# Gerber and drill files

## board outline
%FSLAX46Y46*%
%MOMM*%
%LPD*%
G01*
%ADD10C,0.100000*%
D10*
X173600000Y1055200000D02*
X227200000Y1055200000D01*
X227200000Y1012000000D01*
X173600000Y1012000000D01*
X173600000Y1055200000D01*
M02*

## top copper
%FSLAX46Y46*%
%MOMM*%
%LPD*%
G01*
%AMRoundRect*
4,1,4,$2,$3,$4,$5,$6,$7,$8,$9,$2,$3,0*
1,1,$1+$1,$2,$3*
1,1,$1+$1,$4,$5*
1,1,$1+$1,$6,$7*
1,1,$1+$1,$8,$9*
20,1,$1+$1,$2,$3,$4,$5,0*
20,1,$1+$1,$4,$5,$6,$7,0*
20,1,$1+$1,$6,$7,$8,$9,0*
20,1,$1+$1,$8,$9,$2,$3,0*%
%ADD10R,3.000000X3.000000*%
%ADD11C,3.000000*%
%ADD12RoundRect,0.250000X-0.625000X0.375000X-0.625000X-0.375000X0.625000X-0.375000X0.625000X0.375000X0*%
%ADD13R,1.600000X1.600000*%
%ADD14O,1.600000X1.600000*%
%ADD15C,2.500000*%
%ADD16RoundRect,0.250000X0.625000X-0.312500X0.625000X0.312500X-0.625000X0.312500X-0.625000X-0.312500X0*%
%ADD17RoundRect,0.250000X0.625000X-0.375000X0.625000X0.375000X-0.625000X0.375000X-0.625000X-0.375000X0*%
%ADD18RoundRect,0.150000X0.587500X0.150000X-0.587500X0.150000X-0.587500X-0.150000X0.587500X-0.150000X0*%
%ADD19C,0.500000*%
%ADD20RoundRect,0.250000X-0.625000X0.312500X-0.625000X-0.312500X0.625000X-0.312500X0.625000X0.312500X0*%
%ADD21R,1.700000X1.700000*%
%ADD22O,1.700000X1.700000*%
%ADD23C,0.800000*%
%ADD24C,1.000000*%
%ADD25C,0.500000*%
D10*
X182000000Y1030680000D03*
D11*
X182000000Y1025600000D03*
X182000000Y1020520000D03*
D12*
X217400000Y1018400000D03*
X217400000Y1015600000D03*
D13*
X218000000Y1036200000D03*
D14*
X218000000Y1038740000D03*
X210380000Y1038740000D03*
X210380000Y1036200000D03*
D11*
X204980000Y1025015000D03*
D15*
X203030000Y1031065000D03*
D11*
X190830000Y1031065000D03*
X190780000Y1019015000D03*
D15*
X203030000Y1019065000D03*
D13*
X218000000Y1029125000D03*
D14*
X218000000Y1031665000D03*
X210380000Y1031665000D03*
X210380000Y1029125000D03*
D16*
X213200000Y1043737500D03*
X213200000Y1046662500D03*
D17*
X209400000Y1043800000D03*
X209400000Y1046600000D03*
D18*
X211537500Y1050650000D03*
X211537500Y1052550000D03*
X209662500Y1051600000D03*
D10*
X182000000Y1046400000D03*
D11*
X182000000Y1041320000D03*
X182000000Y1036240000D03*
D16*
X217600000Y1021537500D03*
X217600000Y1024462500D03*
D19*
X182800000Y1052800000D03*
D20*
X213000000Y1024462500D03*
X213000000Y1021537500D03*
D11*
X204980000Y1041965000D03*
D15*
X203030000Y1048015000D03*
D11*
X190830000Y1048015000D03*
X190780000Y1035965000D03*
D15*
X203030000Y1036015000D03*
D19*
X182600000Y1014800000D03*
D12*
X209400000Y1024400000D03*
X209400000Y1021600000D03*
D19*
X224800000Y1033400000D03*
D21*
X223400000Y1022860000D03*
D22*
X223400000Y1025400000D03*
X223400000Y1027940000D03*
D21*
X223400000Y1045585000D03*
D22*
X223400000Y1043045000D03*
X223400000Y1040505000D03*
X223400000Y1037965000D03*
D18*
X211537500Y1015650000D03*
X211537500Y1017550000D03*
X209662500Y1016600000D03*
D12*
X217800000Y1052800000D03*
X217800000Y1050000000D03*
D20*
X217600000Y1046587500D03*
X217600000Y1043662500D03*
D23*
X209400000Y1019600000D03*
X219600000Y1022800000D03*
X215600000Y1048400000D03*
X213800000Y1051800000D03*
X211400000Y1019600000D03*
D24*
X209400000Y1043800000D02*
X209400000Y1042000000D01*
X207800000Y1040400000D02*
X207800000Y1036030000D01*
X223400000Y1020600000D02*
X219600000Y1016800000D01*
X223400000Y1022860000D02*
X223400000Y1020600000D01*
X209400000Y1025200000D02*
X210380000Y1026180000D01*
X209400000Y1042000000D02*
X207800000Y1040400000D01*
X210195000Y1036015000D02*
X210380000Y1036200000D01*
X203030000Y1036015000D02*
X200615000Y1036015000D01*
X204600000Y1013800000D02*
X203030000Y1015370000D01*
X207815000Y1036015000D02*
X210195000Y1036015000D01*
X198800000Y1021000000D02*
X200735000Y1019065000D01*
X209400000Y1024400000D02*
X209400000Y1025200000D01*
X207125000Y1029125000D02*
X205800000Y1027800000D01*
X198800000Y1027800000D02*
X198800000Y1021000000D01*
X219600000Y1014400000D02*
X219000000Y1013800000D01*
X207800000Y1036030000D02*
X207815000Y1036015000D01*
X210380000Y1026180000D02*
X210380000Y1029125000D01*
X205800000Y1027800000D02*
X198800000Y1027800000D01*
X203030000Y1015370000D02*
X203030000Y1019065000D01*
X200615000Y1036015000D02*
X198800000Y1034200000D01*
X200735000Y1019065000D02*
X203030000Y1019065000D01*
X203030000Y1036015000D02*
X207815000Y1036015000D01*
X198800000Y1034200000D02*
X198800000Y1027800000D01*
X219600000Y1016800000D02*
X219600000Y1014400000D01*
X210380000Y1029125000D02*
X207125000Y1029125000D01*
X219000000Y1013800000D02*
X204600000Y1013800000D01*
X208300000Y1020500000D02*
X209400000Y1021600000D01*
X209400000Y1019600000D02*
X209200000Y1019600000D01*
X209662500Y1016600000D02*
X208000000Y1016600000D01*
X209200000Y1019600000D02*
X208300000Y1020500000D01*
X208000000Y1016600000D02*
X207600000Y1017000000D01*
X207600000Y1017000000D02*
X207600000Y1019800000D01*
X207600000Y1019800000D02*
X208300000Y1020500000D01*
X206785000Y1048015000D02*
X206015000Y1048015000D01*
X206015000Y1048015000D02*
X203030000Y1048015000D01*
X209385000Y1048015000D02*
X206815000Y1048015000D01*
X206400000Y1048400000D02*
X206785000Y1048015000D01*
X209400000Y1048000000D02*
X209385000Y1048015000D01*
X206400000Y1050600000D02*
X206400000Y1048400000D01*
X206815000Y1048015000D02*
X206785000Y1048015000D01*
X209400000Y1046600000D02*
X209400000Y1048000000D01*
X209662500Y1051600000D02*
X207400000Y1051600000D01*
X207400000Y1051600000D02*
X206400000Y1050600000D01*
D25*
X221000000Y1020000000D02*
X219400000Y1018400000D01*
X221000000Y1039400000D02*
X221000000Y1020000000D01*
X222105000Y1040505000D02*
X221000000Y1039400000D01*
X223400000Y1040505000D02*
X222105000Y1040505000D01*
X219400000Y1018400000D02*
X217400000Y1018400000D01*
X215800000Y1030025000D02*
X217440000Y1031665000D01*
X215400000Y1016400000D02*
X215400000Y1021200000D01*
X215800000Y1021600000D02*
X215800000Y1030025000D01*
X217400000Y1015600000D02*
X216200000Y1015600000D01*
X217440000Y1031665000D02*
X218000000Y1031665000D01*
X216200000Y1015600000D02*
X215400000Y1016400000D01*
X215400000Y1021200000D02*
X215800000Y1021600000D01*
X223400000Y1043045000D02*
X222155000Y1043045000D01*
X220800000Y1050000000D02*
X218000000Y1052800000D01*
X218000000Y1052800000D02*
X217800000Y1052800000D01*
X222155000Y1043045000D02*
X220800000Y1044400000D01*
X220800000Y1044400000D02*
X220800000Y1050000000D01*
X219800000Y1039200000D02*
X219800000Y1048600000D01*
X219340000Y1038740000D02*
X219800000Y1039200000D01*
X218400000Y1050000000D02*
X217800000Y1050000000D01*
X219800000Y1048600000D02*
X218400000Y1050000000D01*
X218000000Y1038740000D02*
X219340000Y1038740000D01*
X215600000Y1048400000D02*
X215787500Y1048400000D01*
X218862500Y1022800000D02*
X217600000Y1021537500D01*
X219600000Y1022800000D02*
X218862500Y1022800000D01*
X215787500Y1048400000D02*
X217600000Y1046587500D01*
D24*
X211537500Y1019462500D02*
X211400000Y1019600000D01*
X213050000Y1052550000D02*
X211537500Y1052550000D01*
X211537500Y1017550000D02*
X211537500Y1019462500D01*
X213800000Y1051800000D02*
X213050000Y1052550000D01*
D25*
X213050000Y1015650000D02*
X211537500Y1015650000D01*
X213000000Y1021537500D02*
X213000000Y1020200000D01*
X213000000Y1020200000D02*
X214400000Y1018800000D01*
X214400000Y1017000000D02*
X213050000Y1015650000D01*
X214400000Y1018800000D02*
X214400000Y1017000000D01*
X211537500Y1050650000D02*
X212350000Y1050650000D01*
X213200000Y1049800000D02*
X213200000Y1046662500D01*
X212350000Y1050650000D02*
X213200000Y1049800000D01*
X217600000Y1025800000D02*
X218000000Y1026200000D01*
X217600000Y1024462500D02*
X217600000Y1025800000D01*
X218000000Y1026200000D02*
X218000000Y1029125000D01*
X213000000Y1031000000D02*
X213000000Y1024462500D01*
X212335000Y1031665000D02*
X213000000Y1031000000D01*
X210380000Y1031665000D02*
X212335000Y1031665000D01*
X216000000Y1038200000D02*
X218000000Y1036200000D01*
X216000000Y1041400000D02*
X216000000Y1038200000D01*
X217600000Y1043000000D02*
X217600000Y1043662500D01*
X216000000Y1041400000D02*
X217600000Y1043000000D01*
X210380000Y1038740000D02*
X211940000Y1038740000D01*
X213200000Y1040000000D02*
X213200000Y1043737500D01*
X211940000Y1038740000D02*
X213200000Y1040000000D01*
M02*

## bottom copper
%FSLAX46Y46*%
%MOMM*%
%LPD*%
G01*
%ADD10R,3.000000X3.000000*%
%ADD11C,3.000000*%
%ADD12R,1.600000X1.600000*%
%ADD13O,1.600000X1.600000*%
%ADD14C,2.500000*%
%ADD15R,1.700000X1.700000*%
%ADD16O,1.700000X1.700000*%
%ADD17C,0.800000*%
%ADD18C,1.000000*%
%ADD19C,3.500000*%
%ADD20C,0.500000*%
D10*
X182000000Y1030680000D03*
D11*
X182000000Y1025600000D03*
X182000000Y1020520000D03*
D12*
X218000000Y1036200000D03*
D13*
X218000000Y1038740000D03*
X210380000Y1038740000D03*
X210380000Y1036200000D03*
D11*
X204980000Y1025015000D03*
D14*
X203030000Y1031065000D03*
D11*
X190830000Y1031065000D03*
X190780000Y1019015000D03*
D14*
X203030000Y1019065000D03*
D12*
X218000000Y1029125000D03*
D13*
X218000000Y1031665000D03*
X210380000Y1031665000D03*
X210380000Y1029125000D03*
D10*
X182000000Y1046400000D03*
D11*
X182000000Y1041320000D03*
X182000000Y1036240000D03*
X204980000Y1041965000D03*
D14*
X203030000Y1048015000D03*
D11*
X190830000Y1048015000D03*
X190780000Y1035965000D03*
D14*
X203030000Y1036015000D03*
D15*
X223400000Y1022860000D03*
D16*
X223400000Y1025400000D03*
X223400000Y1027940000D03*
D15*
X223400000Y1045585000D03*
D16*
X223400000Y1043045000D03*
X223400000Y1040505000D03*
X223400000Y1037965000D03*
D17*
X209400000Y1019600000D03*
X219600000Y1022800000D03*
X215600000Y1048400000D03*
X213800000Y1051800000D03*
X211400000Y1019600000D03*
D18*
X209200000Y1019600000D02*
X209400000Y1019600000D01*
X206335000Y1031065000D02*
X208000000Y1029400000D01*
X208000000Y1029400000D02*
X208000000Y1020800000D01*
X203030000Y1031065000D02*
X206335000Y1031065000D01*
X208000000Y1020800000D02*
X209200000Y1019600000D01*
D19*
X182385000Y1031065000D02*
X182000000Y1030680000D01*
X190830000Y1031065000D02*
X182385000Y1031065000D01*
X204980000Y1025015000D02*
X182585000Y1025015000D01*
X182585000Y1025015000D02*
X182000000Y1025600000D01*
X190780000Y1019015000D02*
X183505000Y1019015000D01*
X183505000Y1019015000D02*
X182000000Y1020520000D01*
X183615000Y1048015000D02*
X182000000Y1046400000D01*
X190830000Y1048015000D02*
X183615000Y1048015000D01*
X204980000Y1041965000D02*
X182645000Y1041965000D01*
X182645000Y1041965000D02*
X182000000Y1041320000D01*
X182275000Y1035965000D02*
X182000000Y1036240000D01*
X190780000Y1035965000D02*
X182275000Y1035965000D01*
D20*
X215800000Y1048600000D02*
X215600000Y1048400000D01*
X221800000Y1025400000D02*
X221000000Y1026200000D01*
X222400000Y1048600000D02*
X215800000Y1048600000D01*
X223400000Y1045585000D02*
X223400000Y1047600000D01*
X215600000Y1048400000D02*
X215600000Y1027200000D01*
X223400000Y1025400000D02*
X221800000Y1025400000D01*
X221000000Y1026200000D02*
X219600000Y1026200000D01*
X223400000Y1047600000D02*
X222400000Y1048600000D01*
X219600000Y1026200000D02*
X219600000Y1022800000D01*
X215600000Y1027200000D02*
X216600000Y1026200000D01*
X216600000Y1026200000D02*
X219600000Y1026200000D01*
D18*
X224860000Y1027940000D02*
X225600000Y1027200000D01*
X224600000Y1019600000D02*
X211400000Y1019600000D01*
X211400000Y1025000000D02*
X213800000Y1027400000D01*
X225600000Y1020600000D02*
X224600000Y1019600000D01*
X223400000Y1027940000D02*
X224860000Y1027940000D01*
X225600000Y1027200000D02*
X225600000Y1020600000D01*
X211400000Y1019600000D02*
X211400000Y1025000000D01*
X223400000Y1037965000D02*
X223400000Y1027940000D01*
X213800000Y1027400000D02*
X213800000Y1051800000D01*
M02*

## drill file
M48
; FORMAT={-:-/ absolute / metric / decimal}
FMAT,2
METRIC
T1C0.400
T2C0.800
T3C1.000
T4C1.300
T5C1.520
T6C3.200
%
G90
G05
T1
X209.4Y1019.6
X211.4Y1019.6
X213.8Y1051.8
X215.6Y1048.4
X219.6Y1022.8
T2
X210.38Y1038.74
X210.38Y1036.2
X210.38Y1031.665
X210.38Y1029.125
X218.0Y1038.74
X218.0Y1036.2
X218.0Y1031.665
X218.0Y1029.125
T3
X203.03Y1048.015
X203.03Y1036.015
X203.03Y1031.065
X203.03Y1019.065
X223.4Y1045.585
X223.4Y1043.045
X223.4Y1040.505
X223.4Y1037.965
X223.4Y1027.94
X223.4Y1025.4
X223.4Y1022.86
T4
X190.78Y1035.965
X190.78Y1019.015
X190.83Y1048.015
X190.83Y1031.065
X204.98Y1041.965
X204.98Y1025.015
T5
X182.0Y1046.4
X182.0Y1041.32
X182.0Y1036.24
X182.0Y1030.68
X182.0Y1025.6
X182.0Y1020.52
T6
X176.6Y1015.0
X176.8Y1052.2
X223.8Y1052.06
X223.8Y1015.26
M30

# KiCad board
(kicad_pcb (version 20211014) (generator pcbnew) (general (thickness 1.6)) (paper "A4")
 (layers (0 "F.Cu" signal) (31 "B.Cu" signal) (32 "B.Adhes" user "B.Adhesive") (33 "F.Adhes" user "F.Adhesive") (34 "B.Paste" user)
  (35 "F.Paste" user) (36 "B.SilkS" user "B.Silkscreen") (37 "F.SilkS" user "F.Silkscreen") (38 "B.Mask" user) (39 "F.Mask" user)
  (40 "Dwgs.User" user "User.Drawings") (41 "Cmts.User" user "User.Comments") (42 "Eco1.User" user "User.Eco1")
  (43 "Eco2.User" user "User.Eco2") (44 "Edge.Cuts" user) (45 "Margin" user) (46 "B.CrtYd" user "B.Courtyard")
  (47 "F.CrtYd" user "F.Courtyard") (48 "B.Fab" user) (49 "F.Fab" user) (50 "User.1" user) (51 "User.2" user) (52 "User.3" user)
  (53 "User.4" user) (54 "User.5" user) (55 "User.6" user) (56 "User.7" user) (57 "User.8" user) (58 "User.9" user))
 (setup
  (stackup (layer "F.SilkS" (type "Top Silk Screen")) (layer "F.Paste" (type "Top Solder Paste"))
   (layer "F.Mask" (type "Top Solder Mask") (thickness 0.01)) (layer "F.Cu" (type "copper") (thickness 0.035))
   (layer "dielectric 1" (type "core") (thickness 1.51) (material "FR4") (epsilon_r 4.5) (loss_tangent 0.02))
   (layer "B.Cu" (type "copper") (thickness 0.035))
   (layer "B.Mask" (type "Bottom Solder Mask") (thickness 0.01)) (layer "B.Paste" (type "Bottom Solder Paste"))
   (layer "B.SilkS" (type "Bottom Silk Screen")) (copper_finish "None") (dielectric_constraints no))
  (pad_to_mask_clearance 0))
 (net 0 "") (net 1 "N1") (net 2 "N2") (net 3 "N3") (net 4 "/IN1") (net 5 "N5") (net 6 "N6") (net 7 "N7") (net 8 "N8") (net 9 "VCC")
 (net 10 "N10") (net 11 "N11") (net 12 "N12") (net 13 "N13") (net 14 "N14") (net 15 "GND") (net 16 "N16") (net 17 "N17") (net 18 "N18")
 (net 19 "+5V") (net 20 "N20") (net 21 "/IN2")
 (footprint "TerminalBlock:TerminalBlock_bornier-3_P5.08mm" (layer "F.Cu") (at 182 -1030.68 -90)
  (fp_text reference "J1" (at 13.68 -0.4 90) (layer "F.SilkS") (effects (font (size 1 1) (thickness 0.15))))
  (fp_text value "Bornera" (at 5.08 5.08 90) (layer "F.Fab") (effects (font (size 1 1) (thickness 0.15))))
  (pad "1" thru_hole rect (at 0 0 270) (size 3 3) (drill 1.52) (layers *.Cu *.Mask) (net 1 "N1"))
  (pad "2" thru_hole circle (at 5.08 0 270) (size 3 3) (drill 1.52) (layers *.Cu *.Mask) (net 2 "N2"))
  (pad "3" thru_hole circle (at 10.16 0 270) (size 3 3) (drill 1.52) (layers *.Cu *.Mask) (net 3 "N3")))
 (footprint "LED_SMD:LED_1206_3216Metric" (layer "F.Cu") (at 217.4 -1017 -90)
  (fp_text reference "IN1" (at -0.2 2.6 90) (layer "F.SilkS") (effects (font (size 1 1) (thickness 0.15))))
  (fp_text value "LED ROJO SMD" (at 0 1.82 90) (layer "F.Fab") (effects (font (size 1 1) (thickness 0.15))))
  (pad "1" smd roundrect (at -1.4 0 270) (size 1.25 1.75) (layers "F.Cu" "F.Paste" "F.Mask") (roundrect_rratio 0.2) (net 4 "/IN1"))
  (pad "2" smd roundrect (at 1.4 0 270) (size 1.25 1.75) (layers "F.Cu" "F.Paste" "F.Mask") (roundrect_rratio 0.2) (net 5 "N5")))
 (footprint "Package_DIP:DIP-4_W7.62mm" (layer "F.Cu") (at 218 -1036.2 180)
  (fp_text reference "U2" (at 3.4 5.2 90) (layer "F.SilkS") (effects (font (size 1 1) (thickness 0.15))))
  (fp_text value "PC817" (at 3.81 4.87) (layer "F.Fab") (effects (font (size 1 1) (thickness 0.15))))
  (pad "1" thru_hole rect (at 0 0 180) (size 1.6 1.6) (drill 0.8) (layers *.Cu *.Mask) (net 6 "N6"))
  (pad "2" thru_hole oval (at 0 2.54 180) (size 1.6 1.6) (drill 0.8) (layers *.Cu *.Mask) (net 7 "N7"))
  (pad "3" thru_hole oval (at 7.62 2.54 180) (size 1.6 1.6) (drill 0.8) (layers *.Cu *.Mask) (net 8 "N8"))
  (pad "4" thru_hole oval (at 7.62 0 180) (size 1.6 1.6) (drill 0.8) (layers *.Cu *.Mask) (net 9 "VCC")))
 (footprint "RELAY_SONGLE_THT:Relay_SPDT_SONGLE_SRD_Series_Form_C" (layer "F.Cu") (at 204.98 -1025.015 180)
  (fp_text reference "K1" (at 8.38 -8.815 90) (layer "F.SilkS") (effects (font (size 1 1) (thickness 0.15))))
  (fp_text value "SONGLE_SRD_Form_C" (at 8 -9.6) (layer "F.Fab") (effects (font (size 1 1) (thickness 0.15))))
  (pad "1" thru_hole circle (at 0 0 270) (size 3 3) (drill 1.3) (layers *.Cu *.Mask) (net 2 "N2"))
  (pad "2" thru_hole circle (at 1.95 6.05 270) (size 2.5 2.5) (drill 1) (layers *.Cu *.Mask) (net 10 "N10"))
  (pad "3" thru_hole circle (at 14.15 6.05 270) (size 3 3) (drill 1.3) (layers *.Cu *.Mask) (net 1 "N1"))
  (pad "4" thru_hole circle (at 14.2 -6 270) (size 3 3) (drill 1.3) (layers *.Cu *.Mask) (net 3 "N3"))
  (pad "5" thru_hole circle (at 1.95 -5.95 270) (size 2.5 2.5) (drill 1) (layers *.Cu *.Mask) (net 9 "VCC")))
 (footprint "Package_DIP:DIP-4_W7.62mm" (layer "F.Cu") (at 218 -1029.125 180)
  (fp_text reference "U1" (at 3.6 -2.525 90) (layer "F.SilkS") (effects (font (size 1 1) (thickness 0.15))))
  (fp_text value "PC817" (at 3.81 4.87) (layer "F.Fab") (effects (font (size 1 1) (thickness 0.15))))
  (pad "1" thru_hole rect (at 0 0 180) (size 1.6 1.6) (drill 0.8) (layers *.Cu *.Mask) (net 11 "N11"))
  (pad "2" thru_hole oval (at 0 2.54 180) (size 1.6 1.6) (drill 0.8) (layers *.Cu *.Mask) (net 5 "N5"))
  (pad "3" thru_hole oval (at 7.62 2.54 180) (size 1.6 1.6) (drill 0.8) (layers *.Cu *.Mask) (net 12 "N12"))
  (pad "4" thru_hole oval (at 7.62 0 180) (size 1.6 1.6) (drill 0.8) (layers *.Cu *.Mask) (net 9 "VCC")))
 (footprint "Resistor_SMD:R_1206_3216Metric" (layer "F.Cu") (at 213.2 -1045.2 90)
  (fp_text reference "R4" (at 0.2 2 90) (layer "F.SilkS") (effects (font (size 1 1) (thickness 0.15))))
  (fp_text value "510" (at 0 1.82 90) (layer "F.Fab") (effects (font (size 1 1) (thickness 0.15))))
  (pad "1" smd roundrect (at -1.4625 0 90) (size 1.125 1.75) (layers "F.Cu" "F.Paste" "F.Mask") (roundrect_rratio 0.222222) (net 8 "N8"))
  (pad "2" smd roundrect (at 1.4625 0 90) (size 1.125 1.75) (layers "F.Cu" "F.Paste" "F.Mask") (roundrect_rratio 0.222222) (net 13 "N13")))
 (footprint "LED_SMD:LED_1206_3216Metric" (layer "F.Cu") (at 209.4 -1045.2 90)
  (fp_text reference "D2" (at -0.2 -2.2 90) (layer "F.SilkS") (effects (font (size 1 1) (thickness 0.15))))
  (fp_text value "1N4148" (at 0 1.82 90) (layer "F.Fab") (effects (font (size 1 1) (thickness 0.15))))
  (pad "1" smd roundrect (at -1.4 0 90) (size 1.25 1.75) (layers "F.Cu" "F.Paste" "F.Mask") (roundrect_rratio 0.2) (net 9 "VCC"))
  (pad "2" smd roundrect (at 1.4 0 90) (size 1.25 1.75) (layers "F.Cu" "F.Paste" "F.Mask") (roundrect_rratio 0.2) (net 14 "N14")))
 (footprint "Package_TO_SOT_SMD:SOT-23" (layer "F.Cu") (at 210.6 -1051.6 180)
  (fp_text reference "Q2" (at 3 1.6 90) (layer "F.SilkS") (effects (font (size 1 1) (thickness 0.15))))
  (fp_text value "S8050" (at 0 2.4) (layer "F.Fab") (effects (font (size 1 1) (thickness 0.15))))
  (pad "1" smd roundrect (at -0.9375 -0.95 180) (size 1.475 0.6) (layers "F.Cu" "F.Paste" "F.Mask") (roundrect_rratio 0.25) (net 13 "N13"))
  (pad "2" smd roundrect (at -0.9375 0.95 180) (size 1.475 0.6) (layers "F.Cu" "F.Paste" "F.Mask") (roundrect_rratio 0.25) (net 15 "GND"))
  (pad "3" smd roundrect (at 0.9375 0 180) (size 1.475 0.6) (layers "F.Cu" "F.Paste" "F.Mask") (roundrect_rratio 0.25) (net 14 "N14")))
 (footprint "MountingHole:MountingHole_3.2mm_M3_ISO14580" (layer "F.Cu") (at 176.8 -1052.2)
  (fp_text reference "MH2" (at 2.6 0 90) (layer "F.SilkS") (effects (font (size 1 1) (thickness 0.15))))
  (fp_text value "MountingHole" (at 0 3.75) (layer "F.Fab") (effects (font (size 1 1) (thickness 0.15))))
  (pad "" np_thru_hole circle (at 0 0) (size 3.2 3.2) (drill 3.2) (layers *.Cu *.Mask)))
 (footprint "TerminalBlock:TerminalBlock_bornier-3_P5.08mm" (layer "F.Cu") (at 182 -1046.4 -90)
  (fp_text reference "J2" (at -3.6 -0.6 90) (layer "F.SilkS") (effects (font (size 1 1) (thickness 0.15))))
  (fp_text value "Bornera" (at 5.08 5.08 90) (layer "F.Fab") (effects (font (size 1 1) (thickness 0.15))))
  (pad "1" thru_hole rect (at 0 0 270) (size 3 3) (drill 1.52) (layers *.Cu *.Mask) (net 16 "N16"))
  (pad "2" thru_hole circle (at 5.08 0 270) (size 3 3) (drill 1.52) (layers *.Cu *.Mask) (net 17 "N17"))
  (pad "3" thru_hole circle (at 10.16 0 270) (size 3 3) (drill 1.52) (layers *.Cu *.Mask) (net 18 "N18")))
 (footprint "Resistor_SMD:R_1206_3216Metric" (layer "F.Cu") (at 217.6 -1023 90)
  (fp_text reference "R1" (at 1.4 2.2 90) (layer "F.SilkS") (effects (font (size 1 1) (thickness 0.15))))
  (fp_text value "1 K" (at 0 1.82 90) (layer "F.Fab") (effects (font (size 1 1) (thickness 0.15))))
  (pad "1" smd roundrect (at -1.4625 0 90) (size 1.125 1.75) (layers "F.Cu" "F.Paste" "F.Mask") (roundrect_rratio 0.222222) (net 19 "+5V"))
  (pad "2" smd roundrect (at 1.4625 0 90) (size 1.125 1.75) (layers "F.Cu" "F.Paste" "F.Mask") (roundrect_rratio 0.222222) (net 11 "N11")))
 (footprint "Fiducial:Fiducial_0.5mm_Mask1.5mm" (layer "F.Cu") (at 182.8 -1052.8)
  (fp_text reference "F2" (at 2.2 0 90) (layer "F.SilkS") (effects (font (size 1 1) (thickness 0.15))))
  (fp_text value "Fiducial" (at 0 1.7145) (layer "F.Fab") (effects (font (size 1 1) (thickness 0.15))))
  (pad "" smd circle (at 0 0) (size 0.5 0.5) (layers "F.Cu" "F.Mask") (solder_mask_margin 0.5) (clearance 0.5)))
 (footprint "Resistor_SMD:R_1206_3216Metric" (layer "F.Cu") (at 213 -1023 -90)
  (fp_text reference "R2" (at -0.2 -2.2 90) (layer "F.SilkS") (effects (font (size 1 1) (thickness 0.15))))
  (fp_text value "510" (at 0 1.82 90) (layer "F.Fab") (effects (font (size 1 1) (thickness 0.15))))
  (pad "1" smd roundrect (at -1.4625 0 270) (size 1.125 1.75) (layers "F.Cu" "F.Paste" "F.Mask") (roundrect_rratio 0.222222) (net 12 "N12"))
  (pad "2" smd roundrect (at 1.4625 0 270) (size 1.125 1.75) (layers "F.Cu" "F.Paste" "F.Mask") (roundrect_rratio 0.222222) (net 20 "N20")))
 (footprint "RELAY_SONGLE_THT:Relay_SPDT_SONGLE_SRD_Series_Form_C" (layer "F.Cu") (at 204.98 -1041.965 180)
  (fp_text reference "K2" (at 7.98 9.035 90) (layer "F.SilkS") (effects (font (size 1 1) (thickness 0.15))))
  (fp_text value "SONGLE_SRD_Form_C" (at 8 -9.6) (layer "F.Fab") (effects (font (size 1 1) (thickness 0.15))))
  (pad "1" thru_hole circle (at 0 0 270) (size 3 3) (drill 1.3) (layers *.Cu *.Mask) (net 17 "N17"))
  (pad "2" thru_hole circle (at 1.95 6.05 270) (size 2.5 2.5) (drill 1) (layers *.Cu *.Mask) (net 14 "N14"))
  (pad "3" thru_hole circle (at 14.15 6.05 270) (size 3 3) (drill 1.3) (layers *.Cu *.Mask) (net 16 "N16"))
  (pad "4" thru_hole circle (at 14.2 -6 270) (size 3 3) (drill 1.3) (layers *.Cu *.Mask) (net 18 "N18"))
  (pad "5" thru_hole circle (at 1.95 -5.95 270) (size 2.5 2.5) (drill 1) (layers *.Cu *.Mask) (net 9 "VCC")))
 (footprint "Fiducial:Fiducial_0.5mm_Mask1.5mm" (layer "F.Cu") (at 182.6 -1014.8)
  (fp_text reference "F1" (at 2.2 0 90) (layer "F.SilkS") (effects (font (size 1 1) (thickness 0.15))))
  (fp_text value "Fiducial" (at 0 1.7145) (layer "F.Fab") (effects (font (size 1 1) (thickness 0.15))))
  (pad "" smd circle (at 0 0) (size 0.5 0.5) (layers "F.Cu" "F.Mask") (solder_mask_margin 0.5) (clearance 0.5)))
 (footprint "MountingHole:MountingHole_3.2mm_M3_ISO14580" (layer "F.Cu") (at 223.8 -1015.26)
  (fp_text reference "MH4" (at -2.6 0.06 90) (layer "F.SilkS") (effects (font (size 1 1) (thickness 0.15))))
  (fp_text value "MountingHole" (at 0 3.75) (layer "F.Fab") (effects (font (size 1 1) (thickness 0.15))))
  (pad "" np_thru_hole circle (at 0 0) (size 3.2 3.2) (drill 3.2) (layers *.Cu *.Mask)))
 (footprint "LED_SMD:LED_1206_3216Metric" (layer "F.Cu") (at 209.4 -1023 -90)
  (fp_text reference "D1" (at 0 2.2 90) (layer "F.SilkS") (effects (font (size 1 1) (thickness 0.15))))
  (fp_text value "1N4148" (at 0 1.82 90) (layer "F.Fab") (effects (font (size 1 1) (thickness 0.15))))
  (pad "1" smd roundrect (at -1.4 0 270) (size 1.25 1.75) (layers "F.Cu" "F.Paste" "F.Mask") (roundrect_rratio 0.2) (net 9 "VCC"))
  (pad "2" smd roundrect (at 1.4 0 270) (size 1.25 1.75) (layers "F.Cu" "F.Paste" "F.Mask") (roundrect_rratio 0.2) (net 10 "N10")))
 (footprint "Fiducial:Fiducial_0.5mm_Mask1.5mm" (layer "F.Cu") (at 224.8 -1033.4)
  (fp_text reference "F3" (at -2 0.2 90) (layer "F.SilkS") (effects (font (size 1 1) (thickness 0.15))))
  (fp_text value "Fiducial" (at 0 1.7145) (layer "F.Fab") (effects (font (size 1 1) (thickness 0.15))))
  (pad "" smd circle (at 0 0) (size 0.5 0.5) (layers "F.Cu" "F.Mask") (solder_mask_margin 0.5) (clearance 0.5)))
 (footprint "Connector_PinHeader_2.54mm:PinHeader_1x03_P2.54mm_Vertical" (layer "F.Cu") (at 223.4 -1022.86 180)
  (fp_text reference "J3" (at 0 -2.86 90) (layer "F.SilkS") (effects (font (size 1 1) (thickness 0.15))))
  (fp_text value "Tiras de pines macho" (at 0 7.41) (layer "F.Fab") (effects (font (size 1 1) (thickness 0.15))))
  (pad "1" thru_hole rect (at 0 0 180) (size 1.7 1.7) (drill 1) (layers *.Cu *.Mask) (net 9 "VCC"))
  (pad "2" thru_hole oval (at 0 2.54 180) (size 1.7 1.7) (drill 1) (layers *.Cu *.Mask) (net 19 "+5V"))
  (pad "3" thru_hole oval (at 0 5.08 180) (size 1.7 1.7) (drill 1) (layers *.Cu *.Mask) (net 15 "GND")))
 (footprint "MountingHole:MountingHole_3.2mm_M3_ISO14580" (layer "F.Cu") (at 176.6 -1015)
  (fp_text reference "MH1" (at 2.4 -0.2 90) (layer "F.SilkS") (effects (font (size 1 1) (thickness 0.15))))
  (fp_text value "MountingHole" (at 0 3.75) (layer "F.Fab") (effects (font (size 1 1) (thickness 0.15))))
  (pad "" np_thru_hole circle (at 0 0) (size 3.2 3.2) (drill 3.2) (layers *.Cu *.Mask)))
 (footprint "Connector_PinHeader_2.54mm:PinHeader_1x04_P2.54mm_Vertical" (layer "F.Cu") (at 223.4 -1045.585)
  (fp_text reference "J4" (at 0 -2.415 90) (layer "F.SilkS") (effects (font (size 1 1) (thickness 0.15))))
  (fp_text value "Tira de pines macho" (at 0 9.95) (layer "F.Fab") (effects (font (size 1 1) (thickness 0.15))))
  (pad "1" thru_hole rect (at 0 0) (size 1.7 1.7) (drill 1) (layers *.Cu *.Mask) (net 19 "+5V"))
  (pad "2" thru_hole oval (at 0 2.54) (size 1.7 1.7) (drill 1) (layers *.Cu *.Mask) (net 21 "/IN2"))
  (pad "3" thru_hole oval (at 0 5.08) (size 1.7 1.7) (drill 1) (layers *.Cu *.Mask) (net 4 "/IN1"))
  (pad "4" thru_hole oval (at 0 7.62) (size 1.7 1.7) (drill 1) (layers *.Cu *.Mask) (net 15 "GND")))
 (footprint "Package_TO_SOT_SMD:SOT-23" (layer "F.Cu") (at 210.6 -1016.6 180)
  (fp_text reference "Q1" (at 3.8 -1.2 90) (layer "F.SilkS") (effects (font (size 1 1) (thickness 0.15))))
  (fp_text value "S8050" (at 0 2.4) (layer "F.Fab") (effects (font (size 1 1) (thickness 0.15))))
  (pad "1" smd roundrect (at -0.9375 -0.95 180) (size 1.475 0.6) (layers "F.Cu" "F.Paste" "F.Mask") (roundrect_rratio 0.25) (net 20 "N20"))
  (pad "2" smd roundrect (at -0.9375 0.95 180) (size 1.475 0.6) (layers "F.Cu" "F.Paste" "F.Mask") (roundrect_rratio 0.25) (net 15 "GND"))
  (pad "3" smd roundrect (at 0.9375 0 180) (size 1.475 0.6) (layers "F.Cu" "F.Paste" "F.Mask") (roundrect_rratio 0.25) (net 10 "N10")))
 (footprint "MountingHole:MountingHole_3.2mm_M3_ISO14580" (layer "F.Cu") (at 223.8 -1052.06)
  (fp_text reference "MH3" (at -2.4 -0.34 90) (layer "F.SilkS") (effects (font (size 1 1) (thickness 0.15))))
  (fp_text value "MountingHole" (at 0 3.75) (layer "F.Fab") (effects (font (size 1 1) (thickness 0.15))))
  (pad "" np_thru_hole circle (at 0 0) (size 3.2 3.2) (drill 3.2) (layers *.Cu *.Mask)))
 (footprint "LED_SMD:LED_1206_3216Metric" (layer "F.Cu") (at 217.8 -1051.4 -90)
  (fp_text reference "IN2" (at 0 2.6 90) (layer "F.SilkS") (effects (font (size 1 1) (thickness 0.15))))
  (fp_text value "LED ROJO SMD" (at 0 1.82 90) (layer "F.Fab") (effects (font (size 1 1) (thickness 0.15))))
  (pad "1" smd roundrect (at -1.4 0 270) (size 1.25 1.75) (layers "F.Cu" "F.Paste" "F.Mask") (roundrect_rratio 0.2) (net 21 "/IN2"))
  (pad "2" smd roundrect (at 1.4 0 270) (size 1.25 1.75) (layers "F.Cu" "F.Paste" "F.Mask") (roundrect_rratio 0.2) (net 7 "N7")))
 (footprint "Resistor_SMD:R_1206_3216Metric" (layer "F.Cu") (at 217.6 -1045.125 -90)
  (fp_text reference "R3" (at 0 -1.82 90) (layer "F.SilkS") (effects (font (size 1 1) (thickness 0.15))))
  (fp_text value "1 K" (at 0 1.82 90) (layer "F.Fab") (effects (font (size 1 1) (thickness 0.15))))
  (pad "1" smd roundrect (at -1.4625 0 270) (size 1.125 1.75) (layers "F.Cu" "F.Paste" "F.Mask") (roundrect_rratio 0.222222) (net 19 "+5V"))
  (pad "2" smd roundrect (at 1.4625 0 270) (size 1.125 1.75) (layers "F.Cu" "F.Paste" "F.Mask") (roundrect_rratio 0.222222) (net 6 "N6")))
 (gr_rect (start 173.6 -1055.2) (end 227.2 -1012) (layer "Edge.Cuts") (width 0.1) (fill none))
 (segment (start 209.4 -1043.8) (end 209.4 -1042) (width 1) (layer "F.Cu") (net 9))
 (segment (start 207.8 -1040.4) (end 207.8 -1036.03) (width 1) (layer "F.Cu") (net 9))
 (segment (start 223.4 -1020.6) (end 219.6 -1016.8) (width 1) (layer "F.Cu") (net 9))
 (segment (start 223.4 -1022.86) (end 223.4 -1020.6) (width 1) (layer "F.Cu") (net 9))
 (segment (start 209.4 -1025.2) (end 210.38 -1026.18) (width 1) (layer "F.Cu") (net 9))
 (segment (start 209.4 -1042) (end 207.8 -1040.4) (width 1) (layer "F.Cu") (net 9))
 (segment (start 210.195 -1036.015) (end 210.38 -1036.2) (width 1) (layer "F.Cu") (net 9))
 (segment (start 203.03 -1036.015) (end 200.615 -1036.015) (width 1) (layer "F.Cu") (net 9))
 (segment (start 204.6 -1013.8) (end 203.03 -1015.37) (width 1) (layer "F.Cu") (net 9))
 (segment (start 207.815 -1036.015) (end 210.195 -1036.015) (width 1) (layer "F.Cu") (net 9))
 (segment (start 198.8 -1021) (end 200.735 -1019.065) (width 1) (layer "F.Cu") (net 9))
 (segment (start 209.4 -1024.4) (end 209.4 -1025.2) (width 1) (layer "F.Cu") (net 9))
 (segment (start 207.125 -1029.125) (end 205.8 -1027.8) (width 1) (layer "F.Cu") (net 9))
 (segment (start 198.8 -1027.8) (end 198.8 -1021) (width 1) (layer "F.Cu") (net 9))
 (segment (start 219.6 -1014.4) (end 219 -1013.8) (width 1) (layer "F.Cu") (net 9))
 (segment (start 207.8 -1036.03) (end 207.815 -1036.015) (width 1) (layer "F.Cu") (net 9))
 (segment (start 210.38 -1026.18) (end 210.38 -1029.125) (width 1) (layer "F.Cu") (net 9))
 (segment (start 205.8 -1027.8) (end 198.8 -1027.8) (width 1) (layer "F.Cu") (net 9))
 (segment (start 203.03 -1015.37) (end 203.03 -1019.065) (width 1) (layer "F.Cu") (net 9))
 (segment (start 200.615 -1036.015) (end 198.8 -1034.2) (width 1) (layer "F.Cu") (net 9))
 (segment (start 200.735 -1019.065) (end 203.03 -1019.065) (width 1) (layer "F.Cu") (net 9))
 (segment (start 203.03 -1036.015) (end 207.815 -1036.015) (width 1) (layer "F.Cu") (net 9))
 (segment (start 198.8 -1034.2) (end 198.8 -1027.8) (width 1) (layer "F.Cu") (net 9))
 (segment (start 219.6 -1016.8) (end 219.6 -1014.4) (width 1) (layer "F.Cu") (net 9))
 (segment (start 210.38 -1029.125) (end 207.125 -1029.125) (width 1) (layer "F.Cu") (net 9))
 (segment (start 219 -1013.8) (end 204.6 -1013.8) (width 1) (layer "F.Cu") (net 9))
 (segment (start 208.3 -1020.5) (end 209.4 -1021.6) (width 1) (layer "F.Cu") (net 10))
 (segment (start 209.4 -1019.6) (end 209.2 -1019.6) (width 1) (layer "F.Cu") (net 10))
 (segment (start 209.6625 -1016.6) (end 208 -1016.6) (width 1) (layer "F.Cu") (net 10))
 (segment (start 209.2 -1019.6) (end 208.3 -1020.5) (width 1) (layer "F.Cu") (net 10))
 (segment (start 208 -1016.6) (end 207.6 -1017) (width 1) (layer "F.Cu") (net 10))
 (segment (start 207.6 -1017) (end 207.6 -1019.8) (width 1) (layer "F.Cu") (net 10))
 (segment (start 207.6 -1019.8) (end 208.3 -1020.5) (width 1) (layer "F.Cu") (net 10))
 (via (at 209.4 -1019.6) (size 0.8) (drill 0.4) (layers "F.Cu" "B.Cu") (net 10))
 (segment (start 209.2 -1019.6) (end 209.4 -1019.6) (width 1) (layer "B.Cu") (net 10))
 (segment (start 206.335 -1031.065) (end 208 -1029.4) (width 1) (layer "B.Cu") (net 10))
 (segment (start 208 -1029.4) (end 208 -1020.8) (width 1) (layer "B.Cu") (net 10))
 (segment (start 203.03 -1031.065) (end 206.335 -1031.065) (width 1) (layer "B.Cu") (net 10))
 (segment (start 208 -1020.8) (end 209.2 -1019.6) (width 1) (layer "B.Cu") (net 10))
 (segment (start 206.785 -1048.015) (end 206.015 -1048.015) (width 1) (layer "F.Cu") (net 14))
 (segment (start 206.015 -1048.015) (end 203.03 -1048.015) (width 1) (layer "F.Cu") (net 14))
 (segment (start 209.385 -1048.015) (end 206.815 -1048.015) (width 1) (layer "F.Cu") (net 14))
 (segment (start 206.4 -1048.4) (end 206.785 -1048.015) (width 1) (layer "F.Cu") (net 14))
 (segment (start 209.4 -1048) (end 209.385 -1048.015) (width 1) (layer "F.Cu") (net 14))
 (segment (start 206.4 -1050.6) (end 206.4 -1048.4) (width 1) (layer "F.Cu") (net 14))
 (segment (start 206.815 -1048.015) (end 206.785 -1048.015) (width 1) (layer "F.Cu") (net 14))
 (segment (start 209.4 -1046.6) (end 209.4 -1048) (width 1) (layer "F.Cu") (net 14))
 (segment (start 209.6625 -1051.6) (end 207.4 -1051.6) (width 1) (layer "F.Cu") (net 14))
 (segment (start 207.4 -1051.6) (end 206.4 -1050.6) (width 1) (layer "F.Cu") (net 14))
 (segment (start 221 -1020) (end 219.4 -1018.4) (width 0.5) (layer "F.Cu") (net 4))
 (segment (start 221 -1039.4) (end 221 -1020) (width 0.5) (layer "F.Cu") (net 4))
 (segment (start 222.105 -1040.505) (end 221 -1039.4) (width 0.5) (layer "F.Cu") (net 4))
 (segment (start 223.4 -1040.505) (end 222.105 -1040.505) (width 0.5) (layer "F.Cu") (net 4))
 (segment (start 219.4 -1018.4) (end 217.4 -1018.4) (width 0.5) (layer "F.Cu") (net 4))
 (segment (start 215.8 -1030.025) (end 217.44 -1031.665) (width 0.5) (layer "F.Cu") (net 5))
 (segment (start 215.4 -1016.4) (end 215.4 -1021.2) (width 0.5) (layer "F.Cu") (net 5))
 (segment (start 215.8 -1021.6) (end 215.8 -1030.025) (width 0.5) (layer "F.Cu") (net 5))
 (segment (start 217.4 -1015.6) (end 216.2 -1015.6) (width 0.5) (layer "F.Cu") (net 5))
 (segment (start 217.44 -1031.665) (end 218 -1031.665) (width 0.5) (layer "F.Cu") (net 5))
 (segment (start 216.2 -1015.6) (end 215.4 -1016.4) (width 0.5) (layer "F.Cu") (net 5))
 (segment (start 215.4 -1021.2) (end 215.8 -1021.6) (width 0.5) (layer "F.Cu") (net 5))
 (segment (start 223.4 -1043.045) (end 222.155 -1043.045) (width 0.5) (layer "F.Cu") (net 21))
 (segment (start 220.8 -1050) (end 218 -1052.8) (width 0.5) (layer "F.Cu") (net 21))
 (segment (start 218 -1052.8) (end 217.8 -1052.8) (width 0.5) (layer "F.Cu") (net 21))
 (segment (start 222.155 -1043.045) (end 220.8 -1044.4) (width 0.5) (layer "F.Cu") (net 21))
 (segment (start 220.8 -1044.4) (end 220.8 -1050) (width 0.5) (layer "F.Cu") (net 21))
 (segment (start 219.8 -1039.2) (end 219.8 -1048.6) (width 0.5) (layer "F.Cu") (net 7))
 (segment (start 219.34 -1038.74) (end 219.8 -1039.2) (width 0.5) (layer "F.Cu") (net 7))
 (segment (start 218.4 -1050) (end 217.8 -1050) (width 0.5) (layer "F.Cu") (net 7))
 (segment (start 219.8 -1048.6) (end 218.4 -1050) (width 0.5) (layer "F.Cu") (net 7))
 (segment (start 218 -1038.74) (end 219.34 -1038.74) (width 0.5) (layer "F.Cu") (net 7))
 (segment (start 182.385 -1031.065) (end 182 -1030.68) (width 3.5) (layer "B.Cu") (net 1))
 (segment (start 190.83 -1031.065) (end 182.385 -1031.065) (width 3.5) (layer "B.Cu") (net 1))
 (segment (start 204.98 -1025.015) (end 182.585 -1025.015) (width 3.5) (layer "B.Cu") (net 2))
 (segment (start 182.585 -1025.015) (end 182 -1025.6) (width 3.5) (layer "B.Cu") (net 2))
 (segment (start 190.78 -1019.015) (end 183.505 -1019.015) (width 3.5) (layer "B.Cu") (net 3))
 (segment (start 183.505 -1019.015) (end 182 -1020.52) (width 3.5) (layer "B.Cu") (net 3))
 (segment (start 183.615 -1048.015) (end 182 -1046.4) (width 3.5) (layer "B.Cu") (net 16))
 (segment (start 190.83 -1048.015) (end 183.615 -1048.015) (width 3.5) (layer "B.Cu") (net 16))
 (segment (start 204.98 -1041.965) (end 182.645 -1041.965) (width 3.5) (layer "B.Cu") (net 17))
 (segment (start 182.645 -1041.965) (end 182 -1041.32) (width 3.5) (layer "B.Cu") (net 17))
 (segment (start 182.275 -1035.965) (end 182 -1036.24) (width 3.5) (layer "B.Cu") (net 18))
 (segment (start 190.78 -1035.965) (end 182.275 -1035.965) (width 3.5) (layer "B.Cu") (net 18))
 (segment (start 215.6 -1048.4) (end 215.7875 -1048.4) (width 0.5) (layer "F.Cu") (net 19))
 (segment (start 218.8625 -1022.8) (end 217.6 -1021.5375) (width 0.5) (layer "F.Cu") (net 19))
 (segment (start 219.6 -1022.8) (end 218.8625 -1022.8) (width 0.5) (layer "F.Cu") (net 19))
 (segment (start 215.7875 -1048.4) (end 217.6 -1046.5875) (width 0.5) (layer "F.Cu") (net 19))
 (via (at 219.6 -1022.8) (size 0.8) (drill 0.4) (layers "F.Cu" "B.Cu") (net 19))
 (via (at 215.6 -1048.4) (size 0.8) (drill 0.4) (layers "F.Cu" "B.Cu") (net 19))
 (segment (start 215.8 -1048.6) (end 215.6 -1048.4) (width 0.5) (layer "B.Cu") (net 19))
 (segment (start 221.8 -1025.4) (end 221 -1026.2) (width 0.5) (layer "B.Cu") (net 19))
 (segment (start 222.4 -1048.6) (end 215.8 -1048.6) (width 0.5) (layer "B.Cu") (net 19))
 (segment (start 223.4 -1045.585) (end 223.4 -1047.6) (width 0.5) (layer "B.Cu") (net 19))
 (segment (start 215.6 -1048.4) (end 215.6 -1027.2) (width 0.5) (layer "B.Cu") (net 19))
 (segment (start 223.4 -1025.4) (end 221.8 -1025.4) (width 0.5) (layer "B.Cu") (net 19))
 (segment (start 221 -1026.2) (end 219.6 -1026.2) (width 0.5) (layer "B.Cu") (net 19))
 (segment (start 223.4 -1047.6) (end 222.4 -1048.6) (width 0.5) (layer "B.Cu") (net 19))
 (segment (start 219.6 -1026.2) (end 219.6 -1022.8) (width 0.5) (layer "B.Cu") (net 19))
 (segment (start 215.6 -1027.2) (end 216.6 -1026.2) (width 0.5) (layer "B.Cu") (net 19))
 (segment (start 216.6 -1026.2) (end 219.6 -1026.2) (width 0.5) (layer "B.Cu") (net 19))
 (segment (start 211.5375 -1019.4625) (end 211.4 -1019.6) (width 1) (layer "F.Cu") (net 15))
 (segment (start 213.05 -1052.55) (end 211.5375 -1052.55) (width 1) (layer "F.Cu") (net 15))
 (segment (start 211.5375 -1017.55) (end 211.5375 -1019.4625) (width 1) (layer "F.Cu") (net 15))
 (segment (start 213.8 -1051.8) (end 213.05 -1052.55) (width 1) (layer "F.Cu") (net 15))
 (via (at 213.8 -1051.8) (size 0.8) (drill 0.4) (layers "F.Cu" "B.Cu") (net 15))
 (via (at 211.4 -1019.6) (size 0.8) (drill 0.4) (layers "F.Cu" "B.Cu") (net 15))
 (segment (start 224.86 -1027.94) (end 225.6 -1027.2) (width 1) (layer "B.Cu") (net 15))
 (segment (start 224.6 -1019.6) (end 211.4 -1019.6) (width 1) (layer "B.Cu") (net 15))
 (segment (start 211.4 -1025) (end 213.8 -1027.4) (width 1) (layer "B.Cu") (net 15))
 (segment (start 225.6 -1020.6) (end 224.6 -1019.6) (width 1) (layer "B.Cu") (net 15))
 (segment (start 223.4 -1027.94) (end 224.86 -1027.94) (width 1) (layer "B.Cu") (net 15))
 (segment (start 225.6 -1027.2) (end 225.6 -1020.6) (width 1) (layer "B.Cu") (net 15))
 (segment (start 211.4 -1019.6) (end 211.4 -1025) (width 1) (layer "B.Cu") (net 15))
 (segment (start 223.4 -1037.965) (end 223.4 -1027.94) (width 1) (layer "B.Cu") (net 15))
 (segment (start 213.8 -1027.4) (end 213.8 -1051.8) (width 1) (layer "B.Cu") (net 15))
 (segment (start 213.05 -1015.65) (end 211.5375 -1015.65) (width 0.5) (layer "F.Cu") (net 20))
 (segment (start 213 -1021.5375) (end 213 -1020.2) (width 0.5) (layer "F.Cu") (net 20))
 (segment (start 213 -1020.2) (end 214.4 -1018.8) (width 0.5) (layer "F.Cu") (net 20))
 (segment (start 214.4 -1017) (end 213.05 -1015.65) (width 0.5) (layer "F.Cu") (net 20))
 (segment (start 214.4 -1018.8) (end 214.4 -1017) (width 0.5) (layer "F.Cu") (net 20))
 (segment (start 211.5375 -1050.65) (end 212.35 -1050.65) (width 0.5) (layer "F.Cu") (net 13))
 (segment (start 213.2 -1049.8) (end 213.2 -1046.6625) (width 0.5) (layer "F.Cu") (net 13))
 (segment (start 212.35 -1050.65) (end 213.2 -1049.8) (width 0.5) (layer "F.Cu") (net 13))
 (segment (start 217.6 -1025.8) (end 218 -1026.2) (width 0.5) (layer "F.Cu") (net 11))
 (segment (start 217.6 -1024.4625) (end 217.6 -1025.8) (width 0.5) (layer "F.Cu") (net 11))
 (segment (start 218 -1026.2) (end 218 -1029.125) (width 0.5) (layer "F.Cu") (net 11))
 (segment (start 213 -1031) (end 213 -1024.4625) (width 0.5) (layer "F.Cu") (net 12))
 (segment (start 212.335 -1031.665) (end 213 -1031) (width 0.5) (layer "F.Cu") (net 12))
 (segment (start 210.38 -1031.665) (end 212.335 -1031.665) (width 0.5) (layer "F.Cu") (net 12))
 (segment (start 216 -1038.2) (end 218 -1036.2) (width 0.5) (layer "F.Cu") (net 6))
 (segment (start 216 -1041.4) (end 216 -1038.2) (width 0.5) (layer "F.Cu") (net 6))
 (segment (start 217.6 -1043) (end 217.6 -1043.6625) (width 0.5) (layer "F.Cu") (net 6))
 (segment (start 216 -1041.4) (end 217.6 -1043) (width 0.5) (layer "F.Cu") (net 6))
 (segment (start 210.38 -1038.74) (end 211.94 -1038.74) (width 0.5) (layer "F.Cu") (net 8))
 (segment (start 213.2 -1040) (end 213.2 -1043.7375) (width 0.5) (layer "F.Cu") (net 8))
 (segment (start 211.94 -1038.74) (end 213.2 -1040) (width 0.5) (layer "F.Cu") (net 8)))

